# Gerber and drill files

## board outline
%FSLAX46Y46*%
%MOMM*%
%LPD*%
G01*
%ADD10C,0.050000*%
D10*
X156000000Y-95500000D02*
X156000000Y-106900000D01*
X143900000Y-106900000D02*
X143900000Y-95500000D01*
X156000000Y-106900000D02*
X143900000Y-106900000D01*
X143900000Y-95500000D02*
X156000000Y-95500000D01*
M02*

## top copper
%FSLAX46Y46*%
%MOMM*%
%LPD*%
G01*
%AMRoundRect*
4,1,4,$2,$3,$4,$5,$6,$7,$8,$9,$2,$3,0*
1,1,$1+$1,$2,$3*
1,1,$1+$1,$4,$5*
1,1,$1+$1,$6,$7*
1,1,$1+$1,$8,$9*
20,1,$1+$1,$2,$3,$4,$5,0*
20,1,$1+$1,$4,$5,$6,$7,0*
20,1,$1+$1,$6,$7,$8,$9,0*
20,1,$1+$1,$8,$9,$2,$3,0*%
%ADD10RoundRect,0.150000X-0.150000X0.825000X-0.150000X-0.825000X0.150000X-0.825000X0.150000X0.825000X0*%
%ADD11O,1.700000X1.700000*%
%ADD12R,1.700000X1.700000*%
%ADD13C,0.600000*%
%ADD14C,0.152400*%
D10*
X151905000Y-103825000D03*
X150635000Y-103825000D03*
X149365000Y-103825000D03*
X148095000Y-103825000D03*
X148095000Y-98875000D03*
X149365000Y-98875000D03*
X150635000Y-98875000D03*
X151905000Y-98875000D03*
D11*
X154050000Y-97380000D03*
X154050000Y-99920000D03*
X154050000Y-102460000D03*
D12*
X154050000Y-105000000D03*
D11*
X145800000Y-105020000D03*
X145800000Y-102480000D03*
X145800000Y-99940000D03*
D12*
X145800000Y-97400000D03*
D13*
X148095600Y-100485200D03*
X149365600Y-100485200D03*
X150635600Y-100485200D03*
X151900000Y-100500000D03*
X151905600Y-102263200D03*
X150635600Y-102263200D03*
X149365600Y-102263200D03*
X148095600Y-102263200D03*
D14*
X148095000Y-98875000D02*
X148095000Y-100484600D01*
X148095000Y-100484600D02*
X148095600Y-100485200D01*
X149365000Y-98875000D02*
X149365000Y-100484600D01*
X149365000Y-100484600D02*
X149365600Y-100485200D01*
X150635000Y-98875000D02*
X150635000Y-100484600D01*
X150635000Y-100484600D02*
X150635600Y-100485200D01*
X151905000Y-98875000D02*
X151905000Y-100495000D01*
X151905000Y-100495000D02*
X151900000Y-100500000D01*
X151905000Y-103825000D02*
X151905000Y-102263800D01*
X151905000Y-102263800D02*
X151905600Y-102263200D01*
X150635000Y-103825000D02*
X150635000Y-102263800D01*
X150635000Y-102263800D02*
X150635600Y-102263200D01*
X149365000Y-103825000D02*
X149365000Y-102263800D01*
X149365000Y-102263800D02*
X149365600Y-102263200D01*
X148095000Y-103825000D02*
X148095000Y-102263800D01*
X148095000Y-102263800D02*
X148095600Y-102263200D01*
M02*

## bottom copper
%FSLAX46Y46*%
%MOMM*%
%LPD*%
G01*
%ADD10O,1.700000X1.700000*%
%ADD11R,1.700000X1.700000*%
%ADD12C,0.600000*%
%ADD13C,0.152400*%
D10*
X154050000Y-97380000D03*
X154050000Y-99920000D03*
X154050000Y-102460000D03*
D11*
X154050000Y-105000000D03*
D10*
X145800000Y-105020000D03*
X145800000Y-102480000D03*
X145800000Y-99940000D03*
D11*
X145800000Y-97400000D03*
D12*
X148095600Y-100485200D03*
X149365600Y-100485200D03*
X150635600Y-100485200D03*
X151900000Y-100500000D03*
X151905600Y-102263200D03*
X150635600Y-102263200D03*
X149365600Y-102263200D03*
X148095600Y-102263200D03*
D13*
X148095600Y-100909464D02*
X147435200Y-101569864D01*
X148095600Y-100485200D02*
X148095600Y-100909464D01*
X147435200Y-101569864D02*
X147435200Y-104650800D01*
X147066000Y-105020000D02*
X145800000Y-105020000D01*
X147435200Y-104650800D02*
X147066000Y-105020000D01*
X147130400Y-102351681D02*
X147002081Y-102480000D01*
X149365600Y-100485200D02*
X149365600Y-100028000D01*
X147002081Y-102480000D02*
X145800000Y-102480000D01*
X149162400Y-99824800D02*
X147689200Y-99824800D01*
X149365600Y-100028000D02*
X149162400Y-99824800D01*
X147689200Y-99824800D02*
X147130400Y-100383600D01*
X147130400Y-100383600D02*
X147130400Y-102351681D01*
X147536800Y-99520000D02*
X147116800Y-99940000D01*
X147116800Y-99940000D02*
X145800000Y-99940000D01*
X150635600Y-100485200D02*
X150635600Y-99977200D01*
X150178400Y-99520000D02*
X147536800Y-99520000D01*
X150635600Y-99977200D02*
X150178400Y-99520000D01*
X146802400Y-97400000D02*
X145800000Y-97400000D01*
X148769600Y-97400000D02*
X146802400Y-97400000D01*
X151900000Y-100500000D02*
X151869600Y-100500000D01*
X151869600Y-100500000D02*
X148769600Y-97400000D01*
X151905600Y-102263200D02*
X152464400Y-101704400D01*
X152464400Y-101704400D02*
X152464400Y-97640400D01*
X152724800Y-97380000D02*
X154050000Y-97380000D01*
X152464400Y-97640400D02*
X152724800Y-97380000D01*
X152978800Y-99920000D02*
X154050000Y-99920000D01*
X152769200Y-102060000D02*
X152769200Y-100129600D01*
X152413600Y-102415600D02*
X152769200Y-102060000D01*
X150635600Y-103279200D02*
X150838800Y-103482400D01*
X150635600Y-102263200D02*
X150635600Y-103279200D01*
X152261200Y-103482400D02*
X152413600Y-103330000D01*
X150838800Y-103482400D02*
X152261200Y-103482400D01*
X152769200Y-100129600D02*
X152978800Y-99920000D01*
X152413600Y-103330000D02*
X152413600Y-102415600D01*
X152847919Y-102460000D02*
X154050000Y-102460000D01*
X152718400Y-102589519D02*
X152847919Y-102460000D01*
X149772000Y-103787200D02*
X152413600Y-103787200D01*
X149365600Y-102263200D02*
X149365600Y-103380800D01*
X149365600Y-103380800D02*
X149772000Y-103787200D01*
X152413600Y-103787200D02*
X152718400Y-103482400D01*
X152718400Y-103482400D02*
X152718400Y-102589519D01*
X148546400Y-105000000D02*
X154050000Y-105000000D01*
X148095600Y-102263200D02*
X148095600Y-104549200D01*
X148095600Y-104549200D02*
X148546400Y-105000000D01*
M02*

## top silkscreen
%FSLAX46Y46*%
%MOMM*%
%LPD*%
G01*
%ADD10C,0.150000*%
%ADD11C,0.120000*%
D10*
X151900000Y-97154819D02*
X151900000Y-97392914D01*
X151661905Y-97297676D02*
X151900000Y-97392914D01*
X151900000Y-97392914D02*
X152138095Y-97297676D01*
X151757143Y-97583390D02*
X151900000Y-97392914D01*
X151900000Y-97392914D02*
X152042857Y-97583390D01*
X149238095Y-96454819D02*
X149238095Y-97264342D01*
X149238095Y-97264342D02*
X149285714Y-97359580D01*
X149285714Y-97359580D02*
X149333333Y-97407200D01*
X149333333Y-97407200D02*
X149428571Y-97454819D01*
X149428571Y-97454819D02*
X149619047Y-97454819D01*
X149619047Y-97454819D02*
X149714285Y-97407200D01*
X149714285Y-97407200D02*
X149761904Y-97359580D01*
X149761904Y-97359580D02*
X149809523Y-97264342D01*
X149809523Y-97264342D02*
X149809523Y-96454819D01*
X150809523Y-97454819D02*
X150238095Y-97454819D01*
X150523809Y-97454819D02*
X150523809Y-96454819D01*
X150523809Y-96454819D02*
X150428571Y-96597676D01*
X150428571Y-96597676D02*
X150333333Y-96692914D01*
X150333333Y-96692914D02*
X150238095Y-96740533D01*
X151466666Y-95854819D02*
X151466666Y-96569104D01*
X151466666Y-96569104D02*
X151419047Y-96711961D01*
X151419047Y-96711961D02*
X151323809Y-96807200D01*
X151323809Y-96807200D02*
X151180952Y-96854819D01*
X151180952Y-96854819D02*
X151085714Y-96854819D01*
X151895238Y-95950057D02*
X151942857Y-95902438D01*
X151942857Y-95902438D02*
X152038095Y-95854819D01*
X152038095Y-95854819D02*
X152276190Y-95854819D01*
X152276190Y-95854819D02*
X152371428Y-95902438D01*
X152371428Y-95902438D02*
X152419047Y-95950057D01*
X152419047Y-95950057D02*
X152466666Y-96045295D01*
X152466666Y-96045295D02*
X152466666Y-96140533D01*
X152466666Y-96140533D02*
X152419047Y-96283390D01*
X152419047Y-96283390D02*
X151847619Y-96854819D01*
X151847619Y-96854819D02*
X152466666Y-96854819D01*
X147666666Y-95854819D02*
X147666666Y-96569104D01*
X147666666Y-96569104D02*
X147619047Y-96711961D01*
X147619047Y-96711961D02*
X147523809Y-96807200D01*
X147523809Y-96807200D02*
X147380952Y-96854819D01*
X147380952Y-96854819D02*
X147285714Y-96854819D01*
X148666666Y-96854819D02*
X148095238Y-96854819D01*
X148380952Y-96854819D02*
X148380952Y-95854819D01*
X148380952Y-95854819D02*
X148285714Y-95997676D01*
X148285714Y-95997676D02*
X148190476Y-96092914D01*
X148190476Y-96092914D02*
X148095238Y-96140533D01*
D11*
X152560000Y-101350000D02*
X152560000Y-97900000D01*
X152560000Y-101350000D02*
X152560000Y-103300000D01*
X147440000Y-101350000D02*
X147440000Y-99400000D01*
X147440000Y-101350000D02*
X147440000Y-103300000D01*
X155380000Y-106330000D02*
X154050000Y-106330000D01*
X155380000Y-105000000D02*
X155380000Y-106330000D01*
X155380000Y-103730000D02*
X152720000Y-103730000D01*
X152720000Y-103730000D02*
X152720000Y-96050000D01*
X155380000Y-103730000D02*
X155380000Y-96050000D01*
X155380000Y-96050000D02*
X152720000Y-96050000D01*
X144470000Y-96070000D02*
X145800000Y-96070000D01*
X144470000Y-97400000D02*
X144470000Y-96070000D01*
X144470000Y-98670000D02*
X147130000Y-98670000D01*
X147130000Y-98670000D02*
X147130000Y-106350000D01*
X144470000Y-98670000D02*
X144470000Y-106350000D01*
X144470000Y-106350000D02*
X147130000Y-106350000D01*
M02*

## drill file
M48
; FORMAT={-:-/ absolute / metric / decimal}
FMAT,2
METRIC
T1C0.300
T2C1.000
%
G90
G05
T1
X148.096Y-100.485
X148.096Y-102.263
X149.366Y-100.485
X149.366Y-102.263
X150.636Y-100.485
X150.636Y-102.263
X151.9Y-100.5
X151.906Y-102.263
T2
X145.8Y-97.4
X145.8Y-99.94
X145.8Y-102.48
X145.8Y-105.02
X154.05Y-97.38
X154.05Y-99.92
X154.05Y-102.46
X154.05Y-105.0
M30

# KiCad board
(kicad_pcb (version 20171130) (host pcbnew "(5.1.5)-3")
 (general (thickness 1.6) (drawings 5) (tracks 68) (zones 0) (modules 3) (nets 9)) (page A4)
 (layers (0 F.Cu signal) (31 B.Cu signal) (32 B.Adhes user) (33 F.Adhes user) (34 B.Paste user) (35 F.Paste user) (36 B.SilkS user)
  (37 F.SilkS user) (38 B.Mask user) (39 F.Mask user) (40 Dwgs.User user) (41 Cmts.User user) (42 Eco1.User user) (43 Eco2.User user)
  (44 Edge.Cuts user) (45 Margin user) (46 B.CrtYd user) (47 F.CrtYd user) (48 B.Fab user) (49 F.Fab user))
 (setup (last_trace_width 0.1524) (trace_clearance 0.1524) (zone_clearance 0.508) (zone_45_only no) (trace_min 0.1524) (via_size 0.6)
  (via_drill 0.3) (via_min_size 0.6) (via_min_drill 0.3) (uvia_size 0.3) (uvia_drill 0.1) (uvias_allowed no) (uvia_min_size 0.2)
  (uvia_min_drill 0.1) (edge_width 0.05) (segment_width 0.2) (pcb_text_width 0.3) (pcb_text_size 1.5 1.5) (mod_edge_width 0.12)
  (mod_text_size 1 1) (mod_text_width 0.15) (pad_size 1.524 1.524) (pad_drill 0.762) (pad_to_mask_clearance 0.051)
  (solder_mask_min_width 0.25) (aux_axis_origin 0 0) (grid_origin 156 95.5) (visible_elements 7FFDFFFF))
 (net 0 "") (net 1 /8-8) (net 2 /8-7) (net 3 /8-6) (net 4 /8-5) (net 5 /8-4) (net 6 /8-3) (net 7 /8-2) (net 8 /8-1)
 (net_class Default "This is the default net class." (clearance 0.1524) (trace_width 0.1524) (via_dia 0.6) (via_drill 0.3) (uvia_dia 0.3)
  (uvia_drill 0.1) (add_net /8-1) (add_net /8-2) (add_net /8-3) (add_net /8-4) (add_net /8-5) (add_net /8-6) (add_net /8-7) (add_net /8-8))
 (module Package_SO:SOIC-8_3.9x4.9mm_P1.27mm (layer F.Cu) (at 150 101.35 270)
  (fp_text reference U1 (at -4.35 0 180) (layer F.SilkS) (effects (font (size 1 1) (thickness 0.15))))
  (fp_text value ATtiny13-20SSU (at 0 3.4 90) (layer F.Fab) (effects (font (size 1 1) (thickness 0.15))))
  (fp_line (start 0 -2.56) (end -3.45 -2.56) (layer F.SilkS) (width 0.12))
  (fp_line (start 0 -2.56) (end 1.95 -2.56) (layer F.SilkS) (width 0.12))
  (fp_line (start 0 2.56) (end -1.95 2.56) (layer F.SilkS) (width 0.12))
  (fp_line (start 0 2.56) (end 1.95 2.56) (layer F.SilkS) (width 0.12))
  (pad 8 smd roundrect (at 2.475 -1.905 270) (size 1.95 0.6) (layers F.Cu F.Paste F.Mask) (roundrect_rratio 0.25) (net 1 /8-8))
  (pad 7 smd roundrect (at 2.475 -0.635 270) (size 1.95 0.6) (layers F.Cu F.Paste F.Mask) (roundrect_rratio 0.25) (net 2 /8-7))
  (pad 6 smd roundrect (at 2.475 0.635 270) (size 1.95 0.6) (layers F.Cu F.Paste F.Mask) (roundrect_rratio 0.25) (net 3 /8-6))
  (pad 5 smd roundrect (at 2.475 1.905 270) (size 1.95 0.6) (layers F.Cu F.Paste F.Mask) (roundrect_rratio 0.25) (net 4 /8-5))
  (pad 4 smd roundrect (at -2.475 1.905 270) (size 1.95 0.6) (layers F.Cu F.Paste F.Mask) (roundrect_rratio 0.25) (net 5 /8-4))
  (pad 3 smd roundrect (at -2.475 0.635 270) (size 1.95 0.6) (layers F.Cu F.Paste F.Mask) (roundrect_rratio 0.25) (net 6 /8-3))
  (pad 2 smd roundrect (at -2.475 -0.635 270) (size 1.95 0.6) (layers F.Cu F.Paste F.Mask) (roundrect_rratio 0.25) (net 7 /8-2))
  (pad 1 smd roundrect (at -2.475 -1.905 270) (size 1.95 0.6) (layers F.Cu F.Paste F.Mask) (roundrect_rratio 0.25) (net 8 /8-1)))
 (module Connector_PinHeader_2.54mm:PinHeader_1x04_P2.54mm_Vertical (layer F.Cu) (at 154.05 105 180)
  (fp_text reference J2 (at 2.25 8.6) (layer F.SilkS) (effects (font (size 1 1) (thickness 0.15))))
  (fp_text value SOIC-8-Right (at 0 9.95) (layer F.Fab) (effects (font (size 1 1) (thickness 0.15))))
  (fp_line (start -1.33 -1.33) (end 0 -1.33) (layer F.SilkS) (width 0.12))
  (fp_line (start -1.33 0) (end -1.33 -1.33) (layer F.SilkS) (width 0.12))
  (fp_line (start -1.33 1.27) (end 1.33 1.27) (layer F.SilkS) (width 0.12))
  (fp_line (start 1.33 1.27) (end 1.33 8.95) (layer F.SilkS) (width 0.12))
  (fp_line (start -1.33 1.27) (end -1.33 8.95) (layer F.SilkS) (width 0.12))
  (fp_line (start -1.33 8.95) (end 1.33 8.95) (layer F.SilkS) (width 0.12))
  (pad 4 thru_hole oval (at 0 7.62 180) (size 1.7 1.7) (drill 1) (layers *.Cu *.Mask) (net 1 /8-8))
  (pad 3 thru_hole oval (at 0 5.08 180) (size 1.7 1.7) (drill 1) (layers *.Cu *.Mask) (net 2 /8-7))
  (pad 2 thru_hole oval (at 0 2.54 180) (size 1.7 1.7) (drill 1) (layers *.Cu *.Mask) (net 3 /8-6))
  (pad 1 thru_hole rect (at 0 0 180) (size 1.7 1.7) (drill 1) (layers *.Cu *.Mask) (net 4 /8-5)))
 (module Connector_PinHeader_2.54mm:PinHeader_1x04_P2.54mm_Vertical (layer F.Cu) (at 145.8 97.4)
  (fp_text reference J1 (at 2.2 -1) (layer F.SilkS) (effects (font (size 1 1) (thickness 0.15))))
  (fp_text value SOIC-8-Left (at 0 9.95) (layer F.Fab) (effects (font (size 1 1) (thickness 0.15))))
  (fp_line (start -1.33 -1.33) (end 0 -1.33) (layer F.SilkS) (width 0.12))
  (fp_line (start -1.33 0) (end -1.33 -1.33) (layer F.SilkS) (width 0.12))
  (fp_line (start -1.33 1.27) (end 1.33 1.27) (layer F.SilkS) (width 0.12))
  (fp_line (start 1.33 1.27) (end 1.33 8.95) (layer F.SilkS) (width 0.12))
  (fp_line (start -1.33 1.27) (end -1.33 8.95) (layer F.SilkS) (width 0.12))
  (fp_line (start -1.33 8.95) (end 1.33 8.95) (layer F.SilkS) (width 0.12))
  (pad 4 thru_hole oval (at 0 7.62) (size 1.7 1.7) (drill 1) (layers *.Cu *.Mask) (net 5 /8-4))
  (pad 3 thru_hole oval (at 0 5.08) (size 1.7 1.7) (drill 1) (layers *.Cu *.Mask) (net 6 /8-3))
  (pad 2 thru_hole oval (at 0 2.54) (size 1.7 1.7) (drill 1) (layers *.Cu *.Mask) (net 7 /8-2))
  (pad 1 thru_hole rect (at 0 0) (size 1.7 1.7) (drill 1) (layers *.Cu *.Mask) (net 8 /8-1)))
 (gr_line (start 156 95.5) (end 156 106.9) (layer Edge.Cuts) (width 0.05))
 (gr_line (start 143.9 106.9) (end 143.9 95.5) (layer Edge.Cuts) (width 0.05))
 (gr_line (start 156 106.9) (end 143.9 106.9) (layer Edge.Cuts) (width 0.05))
 (gr_line (start 143.9 95.5) (end 156 95.5) (layer Edge.Cuts) (width 0.05))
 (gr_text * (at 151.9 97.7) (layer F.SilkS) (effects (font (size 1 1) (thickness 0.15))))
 (via (at 148.0956 100.4852) (size 0.6) (drill 0.3) (layers F.Cu B.Cu) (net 5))
 (segment (start 148.095 98.875) (end 148.095 100.4846) (width 0.1524) (layer F.Cu) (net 5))
 (segment (start 148.095 100.4846) (end 148.0956 100.4852) (width 0.1524) (layer F.Cu) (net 5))
 (segment (start 148.0956 100.909464) (end 147.4352 101.569864) (width 0.1524) (layer B.Cu) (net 5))
 (segment (start 148.0956 100.4852) (end 148.0956 100.909464) (width 0.1524) (layer B.Cu) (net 5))
 (segment (start 147.4352 101.569864) (end 147.4352 104.6508) (width 0.1524) (layer B.Cu) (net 5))
 (segment (start 147.066 105.02) (end 145.8 105.02) (width 0.1524) (layer B.Cu) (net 5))
 (segment (start 147.4352 104.6508) (end 147.066 105.02) (width 0.1524) (layer B.Cu) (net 5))
 (via (at 149.3656 100.4852) (size 0.6) (drill 0.3) (layers F.Cu B.Cu) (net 6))
 (segment (start 149.365 98.875) (end 149.365 100.4846) (width 0.1524) (layer F.Cu) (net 6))
 (segment (start 149.365 100.4846) (end 149.3656 100.4852) (width 0.1524) (layer F.Cu) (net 6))
 (segment (start 147.1304 102.351681) (end 147.002081 102.48) (width 0.1524) (layer B.Cu) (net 6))
 (segment (start 149.3656 100.4852) (end 149.3656 100.028) (width 0.1524) (layer B.Cu) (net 6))
 (segment (start 147.002081 102.48) (end 145.8 102.48) (width 0.1524) (layer B.Cu) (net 6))
 (segment (start 149.1624 99.8248) (end 147.6892 99.8248) (width 0.1524) (layer B.Cu) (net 6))
 (segment (start 149.3656 100.028) (end 149.1624 99.8248) (width 0.1524) (layer B.Cu) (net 6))
 (segment (start 147.6892 99.8248) (end 147.1304 100.3836) (width 0.1524) (layer B.Cu) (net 6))
 (segment (start 147.1304 100.3836) (end 147.1304 102.351681) (width 0.1524) (layer B.Cu) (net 6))
 (via (at 150.6356 100.4852) (size 0.6) (drill 0.3) (layers F.Cu B.Cu) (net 7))
 (segment (start 150.635 98.875) (end 150.635 100.4846) (width 0.1524) (layer F.Cu) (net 7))
 (segment (start 150.635 100.4846) (end 150.6356 100.4852) (width 0.1524) (layer F.Cu) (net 7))
 (segment (start 147.5368 99.52) (end 147.1168 99.94) (width 0.1524) (layer B.Cu) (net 7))
 (segment (start 147.1168 99.94) (end 145.8 99.94) (width 0.1524) (layer B.Cu) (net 7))
 (segment (start 150.6356 100.4852) (end 150.6356 99.9772) (width 0.1524) (layer B.Cu) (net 7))
 (segment (start 150.1784 99.52) (end 147.5368 99.52) (width 0.1524) (layer B.Cu) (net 7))
 (segment (start 150.6356 99.9772) (end 150.1784 99.52) (width 0.1524) (layer B.Cu) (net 7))
 (segment (start 151.905 98.875) (end 151.905 100.495) (width 0.1524) (layer F.Cu) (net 8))
 (via (at 151.9 100.5) (size 0.6) (drill 0.3) (layers F.Cu B.Cu) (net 8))
 (segment (start 151.905 100.495) (end 151.9 100.5) (width 0.1524) (layer F.Cu) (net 8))
 (segment (start 146.8024 97.4) (end 145.8 97.4) (width 0.1524) (layer B.Cu) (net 8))
 (segment (start 148.7696 97.4) (end 146.8024 97.4) (width 0.1524) (layer B.Cu) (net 8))
 (segment (start 151.9 100.5) (end 151.8696 100.5) (width 0.1524) (layer B.Cu) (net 8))
 (segment (start 151.8696 100.5) (end 148.7696 97.4) (width 0.1524) (layer B.Cu) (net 8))
 (segment (start 151.905 103.825) (end 151.905 102.2638) (width 0.1524) (layer F.Cu) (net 1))
 (via (at 151.9056 102.2632) (size 0.6) (drill 0.3) (layers F.Cu B.Cu) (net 1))
 (segment (start 151.905 102.2638) (end 151.9056 102.2632) (width 0.1524) (layer F.Cu) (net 1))
 (segment (start 151.9056 102.2632) (end 152.4644 101.7044) (width 0.1524) (layer B.Cu) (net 1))
 (segment (start 152.4644 101.7044) (end 152.4644 97.6404) (width 0.1524) (layer B.Cu) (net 1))
 (segment (start 152.7248 97.38) (end 154.05 97.38) (width 0.1524) (layer B.Cu) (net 1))
 (segment (start 152.4644 97.6404) (end 152.7248 97.38) (width 0.1524) (layer B.Cu) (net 1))
 (segment (start 150.635 103.825) (end 150.635 102.2638) (width 0.1524) (layer F.Cu) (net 2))
 (via (at 150.6356 102.2632) (size 0.6) (drill 0.3) (layers F.Cu B.Cu) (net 2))
 (segment (start 150.635 102.2638) (end 150.6356 102.2632) (width 0.1524) (layer F.Cu) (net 2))
 (segment (start 152.9788 99.92) (end 154.05 99.92) (width 0.1524) (layer B.Cu) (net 2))
 (segment (start 152.7692 102.06) (end 152.7692 100.1296) (width 0.1524) (layer B.Cu) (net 2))
 (segment (start 152.4136 102.4156) (end 152.7692 102.06) (width 0.1524) (layer B.Cu) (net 2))
 (segment (start 150.6356 103.2792) (end 150.8388 103.4824) (width 0.1524) (layer B.Cu) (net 2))
 (segment (start 150.6356 102.2632) (end 150.6356 103.2792) (width 0.1524) (layer B.Cu) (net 2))
 (segment (start 152.2612 103.4824) (end 152.4136 103.33) (width 0.1524) (layer B.Cu) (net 2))
 (segment (start 150.8388 103.4824) (end 152.2612 103.4824) (width 0.1524) (layer B.Cu) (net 2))
 (segment (start 152.7692 100.1296) (end 152.9788 99.92) (width 0.1524) (layer B.Cu) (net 2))
 (segment (start 152.4136 103.33) (end 152.4136 102.4156) (width 0.1524) (layer B.Cu) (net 2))
 (via (at 149.3656 102.2632) (size 0.6) (drill 0.3) (layers F.Cu B.Cu) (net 3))
 (segment (start 149.365 103.825) (end 149.365 102.2638) (width 0.1524) (layer F.Cu) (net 3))
 (segment (start 149.365 102.2638) (end 149.3656 102.2632) (width 0.1524) (layer F.Cu) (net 3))
 (segment (start 152.847919 102.46) (end 154.05 102.46) (width 0.1524) (layer B.Cu) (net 3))
 (segment (start 152.7184 102.589519) (end 152.847919 102.46) (width 0.1524) (layer B.Cu) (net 3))
 (segment (start 149.772 103.7872) (end 152.4136 103.7872) (width 0.1524) (layer B.Cu) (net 3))
 (segment (start 149.3656 102.2632) (end 149.3656 103.3808) (width 0.1524) (layer B.Cu) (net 3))
 (segment (start 149.3656 103.3808) (end 149.772 103.7872) (width 0.1524) (layer B.Cu) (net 3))
 (segment (start 152.4136 103.7872) (end 152.7184 103.4824) (width 0.1524) (layer B.Cu) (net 3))
 (segment (start 152.7184 103.4824) (end 152.7184 102.589519) (width 0.1524) (layer B.Cu) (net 3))
 (segment (start 148.095 103.825) (end 148.095 102.2638) (width 0.1524) (layer F.Cu) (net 4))
 (via (at 148.0956 102.2632) (size 0.6) (drill 0.3) (layers F.Cu B.Cu) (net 4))
 (segment (start 148.095 102.2638) (end 148.0956 102.2632) (width 0.1524) (layer F.Cu) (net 4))
 (segment (start 148.5464 105) (end 154.05 105) (width 0.1524) (layer B.Cu) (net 4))
 (segment (start 148.0956 102.2632) (end 148.0956 104.5492) (width 0.1524) (layer B.Cu) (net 4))
 (segment (start 148.0956 104.5492) (end 148.5464 105) (width 0.1524) (layer B.Cu) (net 4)))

